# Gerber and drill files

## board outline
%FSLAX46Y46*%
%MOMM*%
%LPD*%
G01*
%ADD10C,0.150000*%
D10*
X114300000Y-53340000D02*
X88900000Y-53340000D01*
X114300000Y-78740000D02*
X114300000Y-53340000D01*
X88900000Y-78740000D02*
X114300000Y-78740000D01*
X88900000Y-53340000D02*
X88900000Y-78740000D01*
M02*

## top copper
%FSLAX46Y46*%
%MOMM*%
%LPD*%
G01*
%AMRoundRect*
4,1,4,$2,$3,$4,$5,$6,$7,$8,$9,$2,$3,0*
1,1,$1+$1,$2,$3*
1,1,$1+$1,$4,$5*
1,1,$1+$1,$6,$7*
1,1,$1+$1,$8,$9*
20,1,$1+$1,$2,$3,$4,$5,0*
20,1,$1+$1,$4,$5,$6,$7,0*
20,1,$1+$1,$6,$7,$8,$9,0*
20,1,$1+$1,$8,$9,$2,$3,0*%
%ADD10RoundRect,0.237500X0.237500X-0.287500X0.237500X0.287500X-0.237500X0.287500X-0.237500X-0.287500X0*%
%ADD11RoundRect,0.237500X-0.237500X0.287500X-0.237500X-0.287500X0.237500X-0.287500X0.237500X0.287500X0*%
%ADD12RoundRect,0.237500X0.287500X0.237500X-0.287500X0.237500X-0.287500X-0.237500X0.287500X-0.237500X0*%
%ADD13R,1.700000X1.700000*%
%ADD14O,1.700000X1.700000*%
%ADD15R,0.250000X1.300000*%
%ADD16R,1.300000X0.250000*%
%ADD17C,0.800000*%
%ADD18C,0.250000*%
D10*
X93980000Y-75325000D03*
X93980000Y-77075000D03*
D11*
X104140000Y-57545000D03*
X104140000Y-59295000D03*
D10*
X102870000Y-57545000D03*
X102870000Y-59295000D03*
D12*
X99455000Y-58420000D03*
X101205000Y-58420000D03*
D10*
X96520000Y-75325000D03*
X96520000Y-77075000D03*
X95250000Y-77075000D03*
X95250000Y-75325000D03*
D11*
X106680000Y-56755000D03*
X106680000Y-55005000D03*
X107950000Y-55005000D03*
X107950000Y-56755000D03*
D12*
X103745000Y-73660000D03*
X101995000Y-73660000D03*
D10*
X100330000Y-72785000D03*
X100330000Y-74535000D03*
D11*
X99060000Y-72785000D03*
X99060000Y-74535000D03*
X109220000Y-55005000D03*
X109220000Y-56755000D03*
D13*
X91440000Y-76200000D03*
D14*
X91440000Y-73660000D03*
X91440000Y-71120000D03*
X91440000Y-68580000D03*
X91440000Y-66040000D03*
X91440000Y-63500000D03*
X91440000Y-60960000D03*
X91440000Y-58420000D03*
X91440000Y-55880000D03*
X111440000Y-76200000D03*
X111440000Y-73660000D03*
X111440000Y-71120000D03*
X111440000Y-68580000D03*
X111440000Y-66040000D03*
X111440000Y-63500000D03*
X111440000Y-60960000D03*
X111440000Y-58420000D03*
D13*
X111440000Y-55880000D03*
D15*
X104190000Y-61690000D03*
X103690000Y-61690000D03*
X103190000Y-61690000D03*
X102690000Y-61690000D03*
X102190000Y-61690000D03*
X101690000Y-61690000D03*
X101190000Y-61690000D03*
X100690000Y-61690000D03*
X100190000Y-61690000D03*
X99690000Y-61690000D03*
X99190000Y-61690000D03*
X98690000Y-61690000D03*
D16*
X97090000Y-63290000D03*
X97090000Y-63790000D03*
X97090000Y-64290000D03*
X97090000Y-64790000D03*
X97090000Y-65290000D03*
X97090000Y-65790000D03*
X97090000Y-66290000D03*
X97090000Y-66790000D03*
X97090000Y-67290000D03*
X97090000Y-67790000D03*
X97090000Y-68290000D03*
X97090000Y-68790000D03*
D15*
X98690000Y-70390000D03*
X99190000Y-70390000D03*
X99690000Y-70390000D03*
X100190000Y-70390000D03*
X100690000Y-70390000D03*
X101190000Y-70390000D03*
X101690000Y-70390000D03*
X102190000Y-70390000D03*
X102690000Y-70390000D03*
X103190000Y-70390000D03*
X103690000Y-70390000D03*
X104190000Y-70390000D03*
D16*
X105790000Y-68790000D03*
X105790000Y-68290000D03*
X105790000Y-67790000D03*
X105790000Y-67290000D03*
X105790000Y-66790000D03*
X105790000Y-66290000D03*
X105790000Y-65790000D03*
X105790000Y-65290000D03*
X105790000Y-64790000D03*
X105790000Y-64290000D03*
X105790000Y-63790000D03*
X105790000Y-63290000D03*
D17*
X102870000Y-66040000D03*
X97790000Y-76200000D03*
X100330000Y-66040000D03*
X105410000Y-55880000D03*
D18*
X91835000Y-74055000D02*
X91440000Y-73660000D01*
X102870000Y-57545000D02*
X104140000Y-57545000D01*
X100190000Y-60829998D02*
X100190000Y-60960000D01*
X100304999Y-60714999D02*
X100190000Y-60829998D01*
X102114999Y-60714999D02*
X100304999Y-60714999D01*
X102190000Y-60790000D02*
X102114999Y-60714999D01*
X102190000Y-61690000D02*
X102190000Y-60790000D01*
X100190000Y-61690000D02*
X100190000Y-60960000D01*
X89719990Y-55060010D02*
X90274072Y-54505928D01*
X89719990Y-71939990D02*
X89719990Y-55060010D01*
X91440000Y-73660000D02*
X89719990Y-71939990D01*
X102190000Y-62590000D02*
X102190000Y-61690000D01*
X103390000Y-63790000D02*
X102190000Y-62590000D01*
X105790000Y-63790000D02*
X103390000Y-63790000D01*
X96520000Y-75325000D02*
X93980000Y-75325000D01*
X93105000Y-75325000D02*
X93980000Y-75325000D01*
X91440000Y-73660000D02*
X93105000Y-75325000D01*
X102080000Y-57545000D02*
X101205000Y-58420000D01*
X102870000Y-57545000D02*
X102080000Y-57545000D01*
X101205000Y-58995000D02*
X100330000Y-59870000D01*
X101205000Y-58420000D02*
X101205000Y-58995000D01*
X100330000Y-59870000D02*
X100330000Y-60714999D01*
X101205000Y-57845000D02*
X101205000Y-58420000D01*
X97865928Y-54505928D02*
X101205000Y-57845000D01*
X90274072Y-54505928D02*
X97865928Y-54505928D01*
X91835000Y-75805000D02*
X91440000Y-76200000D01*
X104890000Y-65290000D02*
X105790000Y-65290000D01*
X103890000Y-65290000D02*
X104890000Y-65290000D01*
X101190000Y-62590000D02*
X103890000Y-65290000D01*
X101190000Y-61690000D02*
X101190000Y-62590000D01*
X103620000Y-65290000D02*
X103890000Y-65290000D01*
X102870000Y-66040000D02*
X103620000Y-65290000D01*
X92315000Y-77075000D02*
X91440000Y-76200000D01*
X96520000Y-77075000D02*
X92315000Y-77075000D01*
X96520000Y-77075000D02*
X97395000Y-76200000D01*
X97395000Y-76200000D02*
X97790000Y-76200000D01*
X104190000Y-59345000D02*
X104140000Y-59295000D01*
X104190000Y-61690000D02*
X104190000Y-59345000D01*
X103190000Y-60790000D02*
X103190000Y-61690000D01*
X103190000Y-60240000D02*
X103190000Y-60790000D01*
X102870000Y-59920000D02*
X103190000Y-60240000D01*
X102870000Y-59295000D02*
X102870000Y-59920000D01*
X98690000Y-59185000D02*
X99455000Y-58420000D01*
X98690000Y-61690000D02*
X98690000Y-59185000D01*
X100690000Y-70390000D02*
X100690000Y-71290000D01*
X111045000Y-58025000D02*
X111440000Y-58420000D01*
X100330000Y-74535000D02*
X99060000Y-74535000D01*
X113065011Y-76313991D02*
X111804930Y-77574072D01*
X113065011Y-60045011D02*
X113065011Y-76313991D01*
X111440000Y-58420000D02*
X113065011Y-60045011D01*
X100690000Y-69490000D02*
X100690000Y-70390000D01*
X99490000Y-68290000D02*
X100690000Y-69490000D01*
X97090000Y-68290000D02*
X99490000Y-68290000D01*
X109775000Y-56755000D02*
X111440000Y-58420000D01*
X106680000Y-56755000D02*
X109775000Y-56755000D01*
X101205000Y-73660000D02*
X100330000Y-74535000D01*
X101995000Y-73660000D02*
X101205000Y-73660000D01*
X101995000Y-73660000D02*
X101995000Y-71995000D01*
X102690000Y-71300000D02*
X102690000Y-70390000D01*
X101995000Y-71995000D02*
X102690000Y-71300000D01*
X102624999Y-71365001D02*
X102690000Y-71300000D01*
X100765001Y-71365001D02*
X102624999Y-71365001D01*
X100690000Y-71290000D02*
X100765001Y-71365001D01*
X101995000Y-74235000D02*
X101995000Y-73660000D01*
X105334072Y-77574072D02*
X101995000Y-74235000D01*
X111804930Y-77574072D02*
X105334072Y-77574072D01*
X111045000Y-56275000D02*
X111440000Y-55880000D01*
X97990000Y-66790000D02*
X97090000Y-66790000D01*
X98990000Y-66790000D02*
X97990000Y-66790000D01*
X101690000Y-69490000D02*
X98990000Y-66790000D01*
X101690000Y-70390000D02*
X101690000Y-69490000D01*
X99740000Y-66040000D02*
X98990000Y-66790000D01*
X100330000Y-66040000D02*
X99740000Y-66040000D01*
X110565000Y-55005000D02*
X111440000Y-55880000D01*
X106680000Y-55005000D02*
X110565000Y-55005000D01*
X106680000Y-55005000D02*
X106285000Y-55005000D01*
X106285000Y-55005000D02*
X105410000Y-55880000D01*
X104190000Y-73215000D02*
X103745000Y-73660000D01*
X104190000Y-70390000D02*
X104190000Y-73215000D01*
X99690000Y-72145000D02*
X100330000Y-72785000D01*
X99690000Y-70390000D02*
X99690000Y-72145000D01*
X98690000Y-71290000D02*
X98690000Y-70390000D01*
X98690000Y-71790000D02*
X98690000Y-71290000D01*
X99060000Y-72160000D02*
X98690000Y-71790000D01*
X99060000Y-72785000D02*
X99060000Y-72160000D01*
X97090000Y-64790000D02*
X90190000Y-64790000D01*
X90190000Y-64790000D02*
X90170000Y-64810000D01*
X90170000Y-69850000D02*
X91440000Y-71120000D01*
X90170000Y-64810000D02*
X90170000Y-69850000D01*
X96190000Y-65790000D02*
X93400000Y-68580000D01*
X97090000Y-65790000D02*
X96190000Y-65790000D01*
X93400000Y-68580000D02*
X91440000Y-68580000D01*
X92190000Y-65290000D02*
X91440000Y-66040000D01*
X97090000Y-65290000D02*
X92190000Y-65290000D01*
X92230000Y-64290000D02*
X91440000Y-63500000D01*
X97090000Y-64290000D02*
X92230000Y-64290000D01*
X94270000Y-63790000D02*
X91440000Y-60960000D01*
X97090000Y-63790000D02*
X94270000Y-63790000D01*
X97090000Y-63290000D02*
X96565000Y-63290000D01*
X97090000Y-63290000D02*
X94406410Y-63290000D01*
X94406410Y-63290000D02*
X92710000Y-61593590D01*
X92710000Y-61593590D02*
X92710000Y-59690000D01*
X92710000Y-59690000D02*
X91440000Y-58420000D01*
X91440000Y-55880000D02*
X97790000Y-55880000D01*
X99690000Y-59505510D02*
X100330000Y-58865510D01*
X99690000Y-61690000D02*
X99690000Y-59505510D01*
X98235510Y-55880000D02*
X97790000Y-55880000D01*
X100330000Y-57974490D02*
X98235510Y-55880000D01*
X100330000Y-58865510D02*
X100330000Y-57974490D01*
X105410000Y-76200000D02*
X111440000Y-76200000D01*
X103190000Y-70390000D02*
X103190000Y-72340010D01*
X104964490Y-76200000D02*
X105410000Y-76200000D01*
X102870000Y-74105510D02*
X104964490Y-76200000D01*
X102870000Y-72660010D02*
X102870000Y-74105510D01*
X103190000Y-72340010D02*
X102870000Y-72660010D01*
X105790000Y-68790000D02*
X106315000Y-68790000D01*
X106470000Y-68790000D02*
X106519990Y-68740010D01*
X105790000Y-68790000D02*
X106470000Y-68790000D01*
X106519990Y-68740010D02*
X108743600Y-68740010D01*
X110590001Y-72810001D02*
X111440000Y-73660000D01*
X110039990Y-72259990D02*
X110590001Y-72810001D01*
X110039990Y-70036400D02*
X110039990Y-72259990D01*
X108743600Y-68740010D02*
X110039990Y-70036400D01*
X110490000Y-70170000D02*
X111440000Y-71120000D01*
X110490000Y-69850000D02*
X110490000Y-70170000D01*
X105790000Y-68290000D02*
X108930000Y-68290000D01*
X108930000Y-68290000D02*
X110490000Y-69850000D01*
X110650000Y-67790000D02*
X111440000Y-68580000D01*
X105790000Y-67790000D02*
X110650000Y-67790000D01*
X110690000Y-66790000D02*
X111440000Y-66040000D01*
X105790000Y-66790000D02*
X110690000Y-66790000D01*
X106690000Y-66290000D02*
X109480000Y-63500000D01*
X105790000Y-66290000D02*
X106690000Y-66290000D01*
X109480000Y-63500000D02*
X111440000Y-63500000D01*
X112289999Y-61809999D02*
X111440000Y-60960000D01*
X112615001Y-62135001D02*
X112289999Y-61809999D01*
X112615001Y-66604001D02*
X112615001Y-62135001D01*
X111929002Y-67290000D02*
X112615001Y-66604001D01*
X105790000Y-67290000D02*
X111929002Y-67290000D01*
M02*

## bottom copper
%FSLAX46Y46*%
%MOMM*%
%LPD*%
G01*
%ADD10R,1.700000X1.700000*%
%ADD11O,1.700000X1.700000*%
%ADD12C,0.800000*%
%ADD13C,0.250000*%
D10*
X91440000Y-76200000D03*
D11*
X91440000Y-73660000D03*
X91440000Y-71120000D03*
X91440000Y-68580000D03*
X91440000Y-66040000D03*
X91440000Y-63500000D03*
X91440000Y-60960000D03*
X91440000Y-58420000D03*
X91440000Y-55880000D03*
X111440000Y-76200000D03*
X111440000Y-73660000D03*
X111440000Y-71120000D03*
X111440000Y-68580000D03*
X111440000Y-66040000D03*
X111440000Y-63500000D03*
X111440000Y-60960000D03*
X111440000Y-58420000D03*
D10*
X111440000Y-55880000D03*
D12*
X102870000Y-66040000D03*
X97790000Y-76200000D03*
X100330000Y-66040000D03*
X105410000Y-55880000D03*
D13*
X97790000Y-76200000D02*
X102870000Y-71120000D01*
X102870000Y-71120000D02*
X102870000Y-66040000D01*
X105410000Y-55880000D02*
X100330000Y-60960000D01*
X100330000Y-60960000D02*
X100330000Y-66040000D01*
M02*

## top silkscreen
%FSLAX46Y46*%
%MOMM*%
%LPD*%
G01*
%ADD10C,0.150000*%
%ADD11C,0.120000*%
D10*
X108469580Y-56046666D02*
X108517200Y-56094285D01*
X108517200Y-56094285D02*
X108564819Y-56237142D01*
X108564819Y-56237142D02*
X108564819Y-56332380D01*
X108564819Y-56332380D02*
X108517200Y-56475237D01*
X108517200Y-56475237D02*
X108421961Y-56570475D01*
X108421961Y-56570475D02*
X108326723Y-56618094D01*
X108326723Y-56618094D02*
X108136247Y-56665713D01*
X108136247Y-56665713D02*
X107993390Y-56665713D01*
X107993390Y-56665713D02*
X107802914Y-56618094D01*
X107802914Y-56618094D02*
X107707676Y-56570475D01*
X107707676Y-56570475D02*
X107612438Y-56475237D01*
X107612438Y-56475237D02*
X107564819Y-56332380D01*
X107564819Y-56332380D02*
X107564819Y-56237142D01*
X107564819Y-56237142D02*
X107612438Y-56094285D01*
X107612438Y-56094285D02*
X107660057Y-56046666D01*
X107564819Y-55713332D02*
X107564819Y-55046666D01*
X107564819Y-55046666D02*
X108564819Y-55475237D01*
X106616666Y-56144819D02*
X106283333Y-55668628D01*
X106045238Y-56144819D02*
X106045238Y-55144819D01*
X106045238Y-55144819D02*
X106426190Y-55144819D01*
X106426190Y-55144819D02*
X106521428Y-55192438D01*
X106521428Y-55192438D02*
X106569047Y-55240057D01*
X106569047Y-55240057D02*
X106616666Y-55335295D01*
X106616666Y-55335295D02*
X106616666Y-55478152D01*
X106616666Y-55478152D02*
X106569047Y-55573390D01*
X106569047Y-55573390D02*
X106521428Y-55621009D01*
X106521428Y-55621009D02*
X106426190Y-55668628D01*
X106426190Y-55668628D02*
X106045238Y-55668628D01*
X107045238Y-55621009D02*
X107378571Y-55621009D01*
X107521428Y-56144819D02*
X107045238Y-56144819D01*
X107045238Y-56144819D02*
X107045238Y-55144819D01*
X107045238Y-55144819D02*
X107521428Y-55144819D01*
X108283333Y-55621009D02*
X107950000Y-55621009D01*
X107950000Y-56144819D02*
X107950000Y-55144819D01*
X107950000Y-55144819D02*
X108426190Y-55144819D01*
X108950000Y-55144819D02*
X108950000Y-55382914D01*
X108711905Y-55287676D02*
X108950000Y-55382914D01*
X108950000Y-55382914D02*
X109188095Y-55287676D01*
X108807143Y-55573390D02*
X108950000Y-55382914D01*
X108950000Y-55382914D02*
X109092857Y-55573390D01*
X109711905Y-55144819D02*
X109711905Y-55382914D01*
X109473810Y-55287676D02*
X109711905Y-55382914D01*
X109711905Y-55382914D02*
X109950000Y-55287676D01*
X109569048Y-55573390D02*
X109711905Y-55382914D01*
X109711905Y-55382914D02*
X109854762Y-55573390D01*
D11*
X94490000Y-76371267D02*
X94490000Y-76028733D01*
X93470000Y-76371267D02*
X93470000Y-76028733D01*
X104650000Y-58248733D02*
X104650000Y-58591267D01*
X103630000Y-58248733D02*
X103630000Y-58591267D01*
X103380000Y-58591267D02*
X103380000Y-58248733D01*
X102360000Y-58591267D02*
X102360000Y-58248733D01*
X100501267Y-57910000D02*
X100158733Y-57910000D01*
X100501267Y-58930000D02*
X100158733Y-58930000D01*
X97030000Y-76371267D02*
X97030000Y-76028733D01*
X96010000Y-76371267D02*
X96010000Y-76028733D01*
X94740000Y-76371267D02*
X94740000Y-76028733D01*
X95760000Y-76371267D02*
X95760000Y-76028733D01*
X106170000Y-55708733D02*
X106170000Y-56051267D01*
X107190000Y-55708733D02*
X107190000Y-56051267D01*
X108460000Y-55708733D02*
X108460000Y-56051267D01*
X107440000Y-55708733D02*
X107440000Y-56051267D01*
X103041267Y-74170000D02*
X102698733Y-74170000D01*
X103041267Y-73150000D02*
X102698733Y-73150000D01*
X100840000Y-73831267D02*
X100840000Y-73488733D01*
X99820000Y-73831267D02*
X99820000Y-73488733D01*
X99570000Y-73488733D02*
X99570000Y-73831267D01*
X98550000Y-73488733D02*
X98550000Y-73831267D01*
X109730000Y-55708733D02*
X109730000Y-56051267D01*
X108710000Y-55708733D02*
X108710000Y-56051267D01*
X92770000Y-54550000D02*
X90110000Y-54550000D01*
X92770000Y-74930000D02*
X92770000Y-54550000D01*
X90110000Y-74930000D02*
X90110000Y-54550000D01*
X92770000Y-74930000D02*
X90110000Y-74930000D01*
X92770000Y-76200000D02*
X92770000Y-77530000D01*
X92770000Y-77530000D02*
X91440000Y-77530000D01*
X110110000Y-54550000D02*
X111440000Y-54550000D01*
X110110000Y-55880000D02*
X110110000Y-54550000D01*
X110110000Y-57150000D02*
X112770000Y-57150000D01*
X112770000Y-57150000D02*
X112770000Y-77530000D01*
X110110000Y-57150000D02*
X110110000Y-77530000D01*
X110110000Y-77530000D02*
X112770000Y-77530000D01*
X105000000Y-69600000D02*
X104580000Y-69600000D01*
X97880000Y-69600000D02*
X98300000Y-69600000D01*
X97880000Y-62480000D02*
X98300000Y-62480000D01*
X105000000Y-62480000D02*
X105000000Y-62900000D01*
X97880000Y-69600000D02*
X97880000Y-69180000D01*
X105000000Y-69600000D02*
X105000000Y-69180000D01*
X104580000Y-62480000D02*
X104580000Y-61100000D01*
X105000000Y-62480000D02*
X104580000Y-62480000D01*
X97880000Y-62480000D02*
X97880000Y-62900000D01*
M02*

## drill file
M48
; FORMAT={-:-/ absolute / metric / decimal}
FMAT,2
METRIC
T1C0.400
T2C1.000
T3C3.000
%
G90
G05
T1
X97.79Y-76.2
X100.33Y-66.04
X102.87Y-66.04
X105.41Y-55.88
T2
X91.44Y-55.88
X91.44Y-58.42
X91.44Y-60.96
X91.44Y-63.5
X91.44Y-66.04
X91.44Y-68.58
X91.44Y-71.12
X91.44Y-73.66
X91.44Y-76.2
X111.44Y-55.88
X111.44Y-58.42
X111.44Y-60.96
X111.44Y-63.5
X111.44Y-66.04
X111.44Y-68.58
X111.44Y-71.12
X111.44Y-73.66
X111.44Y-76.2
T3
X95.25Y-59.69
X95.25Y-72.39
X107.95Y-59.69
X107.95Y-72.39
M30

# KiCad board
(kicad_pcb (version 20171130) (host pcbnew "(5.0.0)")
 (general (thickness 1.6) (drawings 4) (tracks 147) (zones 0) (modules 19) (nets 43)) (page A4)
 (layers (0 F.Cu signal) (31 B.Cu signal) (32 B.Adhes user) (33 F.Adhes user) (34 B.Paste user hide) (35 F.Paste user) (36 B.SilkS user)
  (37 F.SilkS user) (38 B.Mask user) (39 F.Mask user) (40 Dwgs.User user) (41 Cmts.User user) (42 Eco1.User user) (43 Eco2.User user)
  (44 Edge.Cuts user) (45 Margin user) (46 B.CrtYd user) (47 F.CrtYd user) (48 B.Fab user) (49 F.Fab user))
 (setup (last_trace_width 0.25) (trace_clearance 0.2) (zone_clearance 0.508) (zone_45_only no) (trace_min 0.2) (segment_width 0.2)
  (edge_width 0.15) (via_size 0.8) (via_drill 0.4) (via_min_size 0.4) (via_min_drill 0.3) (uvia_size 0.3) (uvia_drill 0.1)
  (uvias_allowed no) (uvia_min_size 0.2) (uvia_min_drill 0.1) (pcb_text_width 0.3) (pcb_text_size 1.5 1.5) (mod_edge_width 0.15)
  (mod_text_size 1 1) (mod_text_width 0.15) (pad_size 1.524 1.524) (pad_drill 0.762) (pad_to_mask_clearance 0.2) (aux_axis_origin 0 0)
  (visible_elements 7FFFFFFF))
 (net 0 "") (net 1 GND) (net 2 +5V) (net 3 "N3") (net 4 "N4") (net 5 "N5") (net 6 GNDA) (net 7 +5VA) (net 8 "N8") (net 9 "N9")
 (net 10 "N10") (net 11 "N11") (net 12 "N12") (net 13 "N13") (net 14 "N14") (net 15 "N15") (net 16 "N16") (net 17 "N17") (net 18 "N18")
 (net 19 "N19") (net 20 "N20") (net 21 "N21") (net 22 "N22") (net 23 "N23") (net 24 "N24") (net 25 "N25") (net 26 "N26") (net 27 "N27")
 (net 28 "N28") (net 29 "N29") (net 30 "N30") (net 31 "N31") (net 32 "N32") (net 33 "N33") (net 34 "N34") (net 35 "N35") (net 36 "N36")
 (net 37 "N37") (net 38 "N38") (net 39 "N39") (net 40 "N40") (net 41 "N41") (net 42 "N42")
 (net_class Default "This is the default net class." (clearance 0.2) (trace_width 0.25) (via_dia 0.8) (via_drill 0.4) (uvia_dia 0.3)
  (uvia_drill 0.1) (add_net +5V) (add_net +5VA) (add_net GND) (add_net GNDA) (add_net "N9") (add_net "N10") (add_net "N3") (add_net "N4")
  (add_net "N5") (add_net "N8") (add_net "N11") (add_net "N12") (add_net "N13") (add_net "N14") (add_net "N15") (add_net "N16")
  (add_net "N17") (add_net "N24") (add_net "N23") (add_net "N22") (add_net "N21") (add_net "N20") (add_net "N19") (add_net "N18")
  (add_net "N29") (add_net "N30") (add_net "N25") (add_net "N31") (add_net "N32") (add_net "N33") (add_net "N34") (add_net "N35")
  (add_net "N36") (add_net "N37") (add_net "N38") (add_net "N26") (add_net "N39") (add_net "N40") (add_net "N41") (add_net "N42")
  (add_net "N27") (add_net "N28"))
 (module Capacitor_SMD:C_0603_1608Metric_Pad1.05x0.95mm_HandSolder (layer F.Cu) (at 93.98 76.2 90)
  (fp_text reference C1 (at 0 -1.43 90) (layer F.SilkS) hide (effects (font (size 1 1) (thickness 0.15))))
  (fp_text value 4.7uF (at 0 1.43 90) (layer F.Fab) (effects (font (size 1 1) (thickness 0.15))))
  (fp_line (start -0.171267 0.51) (end 0.171267 0.51) (layer F.SilkS) (width 0.12))
  (fp_line (start -0.171267 -0.51) (end 0.171267 -0.51) (layer F.SilkS) (width 0.12))
  (pad 2 smd roundrect (at 0.875 0 90) (size 1.05 0.95) (layers F.Cu F.Paste F.Mask) (roundrect_rratio 0.25) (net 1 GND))
  (pad 1 smd roundrect (at -0.875 0 90) (size 1.05 0.95) (layers F.Cu F.Paste F.Mask) (roundrect_rratio 0.25) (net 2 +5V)))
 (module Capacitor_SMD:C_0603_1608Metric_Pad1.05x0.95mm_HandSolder (layer F.Cu) (at 104.14 58.42 270)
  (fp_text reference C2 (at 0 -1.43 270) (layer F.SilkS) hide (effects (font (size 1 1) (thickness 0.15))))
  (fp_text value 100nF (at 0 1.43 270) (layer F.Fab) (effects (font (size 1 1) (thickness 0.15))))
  (fp_line (start -0.171267 -0.51) (end 0.171267 -0.51) (layer F.SilkS) (width 0.12))
  (fp_line (start -0.171267 0.51) (end 0.171267 0.51) (layer F.SilkS) (width 0.12))
  (pad 1 smd roundrect (at -0.875 0 270) (size 1.05 0.95) (layers F.Cu F.Paste F.Mask) (roundrect_rratio 0.25) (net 1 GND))
  (pad 2 smd roundrect (at 0.875 0 270) (size 1.05 0.95) (layers F.Cu F.Paste F.Mask) (roundrect_rratio 0.25) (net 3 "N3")))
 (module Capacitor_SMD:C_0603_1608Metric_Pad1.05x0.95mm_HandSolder (layer F.Cu) (at 102.87 58.42 90)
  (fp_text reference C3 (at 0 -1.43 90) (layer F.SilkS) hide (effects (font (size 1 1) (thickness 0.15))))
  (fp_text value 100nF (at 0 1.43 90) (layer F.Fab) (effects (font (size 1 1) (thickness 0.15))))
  (fp_line (start -0.171267 0.51) (end 0.171267 0.51) (layer F.SilkS) (width 0.12))
  (fp_line (start -0.171267 -0.51) (end 0.171267 -0.51) (layer F.SilkS) (width 0.12))
  (pad 2 smd roundrect (at 0.875 0 90) (size 1.05 0.95) (layers F.Cu F.Paste F.Mask) (roundrect_rratio 0.25) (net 1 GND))
  (pad 1 smd roundrect (at -0.875 0 90) (size 1.05 0.95) (layers F.Cu F.Paste F.Mask) (roundrect_rratio 0.25) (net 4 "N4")))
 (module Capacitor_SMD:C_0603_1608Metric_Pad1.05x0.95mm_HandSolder (layer F.Cu) (at 100.33 58.42 180)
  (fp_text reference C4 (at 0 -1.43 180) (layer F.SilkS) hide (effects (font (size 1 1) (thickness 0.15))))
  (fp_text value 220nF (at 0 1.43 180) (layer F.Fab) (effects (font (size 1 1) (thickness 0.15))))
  (fp_line (start -0.171267 0.51) (end 0.171267 0.51) (layer F.SilkS) (width 0.12))
  (fp_line (start -0.171267 -0.51) (end 0.171267 -0.51) (layer F.SilkS) (width 0.12))
  (pad 2 smd roundrect (at 0.875 0 180) (size 1.05 0.95) (layers F.Cu F.Paste F.Mask) (roundrect_rratio 0.25) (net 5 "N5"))
  (pad 1 smd roundrect (at -0.875 0 180) (size 1.05 0.95) (layers F.Cu F.Paste F.Mask) (roundrect_rratio 0.25) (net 1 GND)))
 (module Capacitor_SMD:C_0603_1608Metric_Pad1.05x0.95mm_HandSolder (layer F.Cu) (at 96.52 76.2 90)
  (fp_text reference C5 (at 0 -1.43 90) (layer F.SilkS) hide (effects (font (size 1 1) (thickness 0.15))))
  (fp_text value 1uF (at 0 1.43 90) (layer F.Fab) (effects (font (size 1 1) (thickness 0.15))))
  (fp_line (start -0.171267 0.51) (end 0.171267 0.51) (layer F.SilkS) (width 0.12))
  (fp_line (start -0.171267 -0.51) (end 0.171267 -0.51) (layer F.SilkS) (width 0.12))
  (pad 2 smd roundrect (at 0.875 0 90) (size 1.05 0.95) (layers F.Cu F.Paste F.Mask) (roundrect_rratio 0.25) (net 1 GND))
  (pad 1 smd roundrect (at -0.875 0 90) (size 1.05 0.95) (layers F.Cu F.Paste F.Mask) (roundrect_rratio 0.25) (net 2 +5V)))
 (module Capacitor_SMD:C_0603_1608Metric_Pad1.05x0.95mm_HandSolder (layer F.Cu) (at 95.25 76.2 90)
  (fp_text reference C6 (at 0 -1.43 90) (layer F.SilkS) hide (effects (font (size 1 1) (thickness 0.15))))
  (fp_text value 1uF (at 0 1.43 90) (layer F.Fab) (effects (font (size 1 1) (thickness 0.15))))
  (fp_line (start -0.171267 -0.51) (end 0.171267 -0.51) (layer F.SilkS) (width 0.12))
  (fp_line (start -0.171267 0.51) (end 0.171267 0.51) (layer F.SilkS) (width 0.12))
  (pad 1 smd roundrect (at -0.875 0 90) (size 1.05 0.95) (layers F.Cu F.Paste F.Mask) (roundrect_rratio 0.25) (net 2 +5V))
  (pad 2 smd roundrect (at 0.875 0 90) (size 1.05 0.95) (layers F.Cu F.Paste F.Mask) (roundrect_rratio 0.25) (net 1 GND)))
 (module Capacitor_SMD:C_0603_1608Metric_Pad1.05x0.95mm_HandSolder (layer F.Cu) (at 106.68 55.88 270)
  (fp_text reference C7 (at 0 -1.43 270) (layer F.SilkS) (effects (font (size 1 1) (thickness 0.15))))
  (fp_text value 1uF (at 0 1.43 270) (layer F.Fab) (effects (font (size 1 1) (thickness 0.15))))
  (fp_line (start -0.171267 0.51) (end 0.171267 0.51) (layer F.SilkS) (width 0.12))
  (fp_line (start -0.171267 -0.51) (end 0.171267 -0.51) (layer F.SilkS) (width 0.12))
  (pad 2 smd roundrect (at 0.875 0 270) (size 1.05 0.95) (layers F.Cu F.Paste F.Mask) (roundrect_rratio 0.25) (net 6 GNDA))
  (pad 1 smd roundrect (at -0.875 0 270) (size 1.05 0.95) (layers F.Cu F.Paste F.Mask) (roundrect_rratio 0.25) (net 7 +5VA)))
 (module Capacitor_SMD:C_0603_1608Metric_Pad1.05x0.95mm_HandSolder (layer F.Cu) (at 107.95 55.88 270)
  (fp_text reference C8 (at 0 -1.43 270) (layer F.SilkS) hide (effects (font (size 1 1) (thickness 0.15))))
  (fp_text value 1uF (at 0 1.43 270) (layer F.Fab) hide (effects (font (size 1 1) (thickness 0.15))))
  (fp_line (start -0.171267 -0.51) (end 0.171267 -0.51) (layer F.SilkS) (width 0.12))
  (fp_line (start -0.171267 0.51) (end 0.171267 0.51) (layer F.SilkS) (width 0.12))
  (pad 1 smd roundrect (at -0.875 0 270) (size 1.05 0.95) (layers F.Cu F.Paste F.Mask) (roundrect_rratio 0.25) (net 7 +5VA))
  (pad 2 smd roundrect (at 0.875 0 270) (size 1.05 0.95) (layers F.Cu F.Paste F.Mask) (roundrect_rratio 0.25) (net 6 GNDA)))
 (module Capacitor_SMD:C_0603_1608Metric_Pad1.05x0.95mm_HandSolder (layer F.Cu) (at 102.87 73.66 180)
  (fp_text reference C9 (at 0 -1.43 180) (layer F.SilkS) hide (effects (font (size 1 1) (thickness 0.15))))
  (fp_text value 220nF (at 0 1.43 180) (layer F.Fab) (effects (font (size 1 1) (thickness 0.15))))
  (fp_line (start -0.171267 -0.51) (end 0.171267 -0.51) (layer F.SilkS) (width 0.12))
  (fp_line (start -0.171267 0.51) (end 0.171267 0.51) (layer F.SilkS) (width 0.12))
  (pad 1 smd roundrect (at -0.875 0 180) (size 1.05 0.95) (layers F.Cu F.Paste F.Mask) (roundrect_rratio 0.25) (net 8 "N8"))
  (pad 2 smd roundrect (at 0.875 0 180) (size 1.05 0.95) (layers F.Cu F.Paste F.Mask) (roundrect_rratio 0.25) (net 6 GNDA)))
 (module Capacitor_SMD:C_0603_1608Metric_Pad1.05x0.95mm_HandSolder (layer F.Cu) (at 100.33 73.66 90)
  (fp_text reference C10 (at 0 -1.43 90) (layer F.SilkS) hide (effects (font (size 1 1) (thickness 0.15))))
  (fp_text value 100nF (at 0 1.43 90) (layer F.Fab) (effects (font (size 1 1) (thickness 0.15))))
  (fp_line (start -0.171267 0.51) (end 0.171267 0.51) (layer F.SilkS) (width 0.12))
  (fp_line (start -0.171267 -0.51) (end 0.171267 -0.51) (layer F.SilkS) (width 0.12))
  (pad 2 smd roundrect (at 0.875 0 90) (size 1.05 0.95) (layers F.Cu F.Paste F.Mask) (roundrect_rratio 0.25) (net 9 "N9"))
  (pad 1 smd roundrect (at -0.875 0 90) (size 1.05 0.95) (layers F.Cu F.Paste F.Mask) (roundrect_rratio 0.25) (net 6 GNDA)))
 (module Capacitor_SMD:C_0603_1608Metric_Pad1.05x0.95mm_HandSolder (layer F.Cu) (at 99.06 73.66 270)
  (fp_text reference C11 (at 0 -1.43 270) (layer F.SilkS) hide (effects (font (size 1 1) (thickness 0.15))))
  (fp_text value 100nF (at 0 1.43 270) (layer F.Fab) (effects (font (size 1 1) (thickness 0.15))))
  (fp_line (start -0.171267 -0.51) (end 0.171267 -0.51) (layer F.SilkS) (width 0.12))
  (fp_line (start -0.171267 0.51) (end 0.171267 0.51) (layer F.SilkS) (width 0.12))
  (pad 1 smd roundrect (at -0.875 0 270) (size 1.05 0.95) (layers F.Cu F.Paste F.Mask) (roundrect_rratio 0.25) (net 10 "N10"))
  (pad 2 smd roundrect (at 0.875 0 270) (size 1.05 0.95) (layers F.Cu F.Paste F.Mask) (roundrect_rratio 0.25) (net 6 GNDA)))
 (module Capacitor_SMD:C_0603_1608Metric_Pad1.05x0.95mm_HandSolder (layer F.Cu) (at 109.22 55.88 270)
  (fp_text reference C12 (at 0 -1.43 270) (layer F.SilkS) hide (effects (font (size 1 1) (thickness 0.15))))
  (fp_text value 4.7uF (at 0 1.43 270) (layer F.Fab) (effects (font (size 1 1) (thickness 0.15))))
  (fp_line (start -0.171267 -0.51) (end 0.171267 -0.51) (layer F.SilkS) (width 0.12))
  (fp_line (start -0.171267 0.51) (end 0.171267 0.51) (layer F.SilkS) (width 0.12))
  (pad 1 smd roundrect (at -0.875 0 270) (size 1.05 0.95) (layers F.Cu F.Paste F.Mask) (roundrect_rratio 0.25) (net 7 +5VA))
  (pad 2 smd roundrect (at 0.875 0 270) (size 1.05 0.95) (layers F.Cu F.Paste F.Mask) (roundrect_rratio 0.25) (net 6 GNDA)))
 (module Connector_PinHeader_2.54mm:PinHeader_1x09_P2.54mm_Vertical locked (layer F.Cu) (at 91.44 76.2 180)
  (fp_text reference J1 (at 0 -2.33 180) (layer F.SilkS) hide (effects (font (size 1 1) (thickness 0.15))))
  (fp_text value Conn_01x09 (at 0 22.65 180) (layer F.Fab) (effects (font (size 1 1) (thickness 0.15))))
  (fp_line (start -1.33 21.65) (end 1.33 21.65) (layer F.SilkS) (width 0.12))
  (fp_line (start -1.33 1.27) (end -1.33 21.65) (layer F.SilkS) (width 0.12))
  (fp_line (start 1.33 1.27) (end 1.33 21.65) (layer F.SilkS) (width 0.12))
  (fp_line (start -1.33 1.27) (end 1.33 1.27) (layer F.SilkS) (width 0.12))
  (fp_line (start -1.33 0) (end -1.33 -1.33) (layer F.SilkS) (width 0.12))
  (fp_line (start -1.33 -1.33) (end 0 -1.33) (layer F.SilkS) (width 0.12))
  (pad 1 thru_hole rect (at 0 0 180) (size 1.7 1.7) (drill 1) (layers *.Cu *.Mask) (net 2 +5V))
  (pad 2 thru_hole oval (at 0 2.54 180) (size 1.7 1.7) (drill 1) (layers *.Cu *.Mask) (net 1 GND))
  (pad 3 thru_hole oval (at 0 5.08 180) (size 1.7 1.7) (drill 1) (layers *.Cu *.Mask) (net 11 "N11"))
  (pad 4 thru_hole oval (at 0 7.62 180) (size 1.7 1.7) (drill 1) (layers *.Cu *.Mask) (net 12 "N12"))
  (pad 5 thru_hole oval (at 0 10.16 180) (size 1.7 1.7) (drill 1) (layers *.Cu *.Mask) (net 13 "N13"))
  (pad 6 thru_hole oval (at 0 12.7 180) (size 1.7 1.7) (drill 1) (layers *.Cu *.Mask) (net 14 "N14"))
  (pad 7 thru_hole oval (at 0 15.24 180) (size 1.7 1.7) (drill 1) (layers *.Cu *.Mask) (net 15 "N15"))
  (pad 8 thru_hole oval (at 0 17.78 180) (size 1.7 1.7) (drill 1) (layers *.Cu *.Mask) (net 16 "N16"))
  (pad 9 thru_hole oval (at 0 20.32 180) (size 1.7 1.7) (drill 1) (layers *.Cu *.Mask) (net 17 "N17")))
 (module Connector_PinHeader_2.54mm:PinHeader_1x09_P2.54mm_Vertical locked (layer F.Cu) (at 111.44 55.88)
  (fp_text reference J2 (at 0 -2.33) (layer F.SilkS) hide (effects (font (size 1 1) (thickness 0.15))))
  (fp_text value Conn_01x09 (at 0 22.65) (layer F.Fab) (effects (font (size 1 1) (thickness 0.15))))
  (fp_line (start -1.33 -1.33) (end 0 -1.33) (layer F.SilkS) (width 0.12))
  (fp_line (start -1.33 0) (end -1.33 -1.33) (layer F.SilkS) (width 0.12))
  (fp_line (start -1.33 1.27) (end 1.33 1.27) (layer F.SilkS) (width 0.12))
  (fp_line (start 1.33 1.27) (end 1.33 21.65) (layer F.SilkS) (width 0.12))
  (fp_line (start -1.33 1.27) (end -1.33 21.65) (layer F.SilkS) (width 0.12))
  (fp_line (start -1.33 21.65) (end 1.33 21.65) (layer F.SilkS) (width 0.12))
  (pad 9 thru_hole oval (at 0 20.32) (size 1.7 1.7) (drill 1) (layers *.Cu *.Mask) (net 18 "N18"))
  (pad 8 thru_hole oval (at 0 17.78) (size 1.7 1.7) (drill 1) (layers *.Cu *.Mask) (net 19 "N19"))
  (pad 7 thru_hole oval (at 0 15.24) (size 1.7 1.7) (drill 1) (layers *.Cu *.Mask) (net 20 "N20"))
  (pad 6 thru_hole oval (at 0 12.7) (size 1.7 1.7) (drill 1) (layers *.Cu *.Mask) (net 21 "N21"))
  (pad 5 thru_hole oval (at 0 10.16) (size 1.7 1.7) (drill 1) (layers *.Cu *.Mask) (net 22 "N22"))
  (pad 4 thru_hole oval (at 0 7.62) (size 1.7 1.7) (drill 1) (layers *.Cu *.Mask) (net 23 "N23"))
  (pad 3 thru_hole oval (at 0 5.08) (size 1.7 1.7) (drill 1) (layers *.Cu *.Mask) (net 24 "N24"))
  (pad 2 thru_hole oval (at 0 2.54) (size 1.7 1.7) (drill 1) (layers *.Cu *.Mask) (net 6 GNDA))
  (pad 1 thru_hole rect (at 0 0) (size 1.7 1.7) (drill 1) (layers *.Cu *.Mask) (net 7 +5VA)))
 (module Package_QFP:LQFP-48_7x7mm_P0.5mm (layer F.Cu) (at 101.44 66.04 270)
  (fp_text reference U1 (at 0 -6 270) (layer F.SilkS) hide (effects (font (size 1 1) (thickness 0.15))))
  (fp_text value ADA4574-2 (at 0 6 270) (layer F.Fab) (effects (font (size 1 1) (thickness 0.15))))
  (fp_line (start 3.56 -3.56) (end 3.56 -3.14) (layer F.SilkS) (width 0.12))
  (fp_line (start 3.56 3.56) (end 3.56 3.14) (layer F.SilkS) (width 0.12))
  (fp_line (start -3.56 3.56) (end -3.56 3.14) (layer F.SilkS) (width 0.12))
  (fp_line (start -3.56 -3.56) (end -3.14 -3.56) (layer F.SilkS) (width 0.12))
  (fp_line (start 3.56 3.56) (end 3.14 3.56) (layer F.SilkS) (width 0.12))
  (fp_line (start 3.56 -3.56) (end 3.14 -3.56) (layer F.SilkS) (width 0.12))
  (fp_line (start -3.56 -3.14) (end -4.94 -3.14) (layer F.SilkS) (width 0.12))
  (fp_line (start -3.56 -3.56) (end -3.56 -3.14) (layer F.SilkS) (width 0.12))
  (fp_line (start -3.56 3.56) (end -3.14 3.56) (layer F.SilkS) (width 0.12))
  (pad 1 smd rect (at -4.35 -2.75 270) (size 1.3 0.25) (layers F.Cu F.Paste F.Mask) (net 3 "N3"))
  (pad 2 smd rect (at -4.35 -2.25 270) (size 1.3 0.25) (layers F.Cu F.Paste F.Mask) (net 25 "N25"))
  (pad 3 smd rect (at -4.35 -1.75 270) (size 1.3 0.25) (layers F.Cu F.Paste F.Mask) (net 4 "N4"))
  (pad 4 smd rect (at -4.35 -1.25 270) (size 1.3 0.25) (layers F.Cu F.Paste F.Mask) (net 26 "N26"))
  (pad 5 smd rect (at -4.35 -0.75 270) (size 1.3 0.25) (layers F.Cu F.Paste F.Mask) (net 1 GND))
  (pad 6 smd rect (at -4.35 -0.25 270) (size 1.3 0.25) (layers F.Cu F.Paste F.Mask) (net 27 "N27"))
  (pad 7 smd rect (at -4.35 0.25 270) (size 1.3 0.25) (layers F.Cu F.Paste F.Mask) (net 2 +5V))
  (pad 8 smd rect (at -4.35 0.75 270) (size 1.3 0.25) (layers F.Cu F.Paste F.Mask) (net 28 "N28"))
  (pad 9 smd rect (at -4.35 1.25 270) (size 1.3 0.25) (layers F.Cu F.Paste F.Mask) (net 1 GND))
  (pad 10 smd rect (at -4.35 1.75 270) (size 1.3 0.25) (layers F.Cu F.Paste F.Mask) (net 17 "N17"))
  (pad 11 smd rect (at -4.35 2.25 270) (size 1.3 0.25) (layers F.Cu F.Paste F.Mask) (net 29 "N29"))
  (pad 12 smd rect (at -4.35 2.75 270) (size 1.3 0.25) (layers F.Cu F.Paste F.Mask) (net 5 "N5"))
  (pad 13 smd rect (at -2.75 4.35) (size 1.3 0.25) (layers F.Cu F.Paste F.Mask) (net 16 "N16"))
  (pad 14 smd rect (at -2.25 4.35) (size 1.3 0.25) (layers F.Cu F.Paste F.Mask) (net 15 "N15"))
  (pad 15 smd rect (at -1.75 4.35) (size 1.3 0.25) (layers F.Cu F.Paste F.Mask) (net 14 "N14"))
  (pad 16 smd rect (at -1.25 4.35) (size 1.3 0.25) (layers F.Cu F.Paste F.Mask) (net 11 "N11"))
  (pad 17 smd rect (at -0.75 4.35) (size 1.3 0.25) (layers F.Cu F.Paste F.Mask) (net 13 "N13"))
  (pad 18 smd rect (at -0.25 4.35) (size 1.3 0.25) (layers F.Cu F.Paste F.Mask) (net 12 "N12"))
  (pad 19 smd rect (at 0.25 4.35) (size 1.3 0.25) (layers F.Cu F.Paste F.Mask) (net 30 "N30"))
  (pad 20 smd rect (at 0.75 4.35) (size 1.3 0.25) (layers F.Cu F.Paste F.Mask) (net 7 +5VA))
  (pad 21 smd rect (at 1.25 4.35) (size 1.3 0.25) (layers F.Cu F.Paste F.Mask) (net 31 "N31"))
  (pad 22 smd rect (at 1.75 4.35) (size 1.3 0.25) (layers F.Cu F.Paste F.Mask) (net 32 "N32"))
  (pad 23 smd rect (at 2.25 4.35) (size 1.3 0.25) (layers F.Cu F.Paste F.Mask) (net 6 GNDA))
  (pad 24 smd rect (at 2.75 4.35) (size 1.3 0.25) (layers F.Cu F.Paste F.Mask) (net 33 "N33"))
  (pad 25 smd rect (at 4.35 2.75 270) (size 1.3 0.25) (layers F.Cu F.Paste F.Mask) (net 10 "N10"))
  (pad 26 smd rect (at 4.35 2.25 270) (size 1.3 0.25) (layers F.Cu F.Paste F.Mask) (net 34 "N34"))
  (pad 27 smd rect (at 4.35 1.75 270) (size 1.3 0.25) (layers F.Cu F.Paste F.Mask) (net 9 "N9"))
  (pad 28 smd rect (at 4.35 1.25 270) (size 1.3 0.25) (layers F.Cu F.Paste F.Mask) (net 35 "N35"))
  (pad 29 smd rect (at 4.35 0.75 270) (size 1.3 0.25) (layers F.Cu F.Paste F.Mask) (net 6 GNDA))
  (pad 30 smd rect (at 4.35 0.25 270) (size 1.3 0.25) (layers F.Cu F.Paste F.Mask) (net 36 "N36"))
  (pad 31 smd rect (at 4.35 -0.25 270) (size 1.3 0.25) (layers F.Cu F.Paste F.Mask) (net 7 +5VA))
  (pad 32 smd rect (at 4.35 -0.75 270) (size 1.3 0.25) (layers F.Cu F.Paste F.Mask) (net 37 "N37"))
  (pad 33 smd rect (at 4.35 -1.25 270) (size 1.3 0.25) (layers F.Cu F.Paste F.Mask) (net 6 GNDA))
  (pad 34 smd rect (at 4.35 -1.75 270) (size 1.3 0.25) (layers F.Cu F.Paste F.Mask) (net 18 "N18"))
  (pad 35 smd rect (at 4.35 -2.25 270) (size 1.3 0.25) (layers F.Cu F.Paste F.Mask) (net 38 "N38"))
  (pad 36 smd rect (at 4.35 -2.75 270) (size 1.3 0.25) (layers F.Cu F.Paste F.Mask) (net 8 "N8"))
  (pad 37 smd rect (at 2.75 -4.35) (size 1.3 0.25) (layers F.Cu F.Paste F.Mask) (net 19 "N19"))
  (pad 38 smd rect (at 2.25 -4.35) (size 1.3 0.25) (layers F.Cu F.Paste F.Mask) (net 20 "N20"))
  (pad 39 smd rect (at 1.75 -4.35) (size 1.3 0.25) (layers F.Cu F.Paste F.Mask) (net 21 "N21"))
  (pad 40 smd rect (at 1.25 -4.35) (size 1.3 0.25) (layers F.Cu F.Paste F.Mask) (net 24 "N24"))
  (pad 41 smd rect (at 0.75 -4.35) (size 1.3 0.25) (layers F.Cu F.Paste F.Mask) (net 22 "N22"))
  (pad 42 smd rect (at 0.25 -4.35) (size 1.3 0.25) (layers F.Cu F.Paste F.Mask) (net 23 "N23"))
  (pad 43 smd rect (at -0.25 -4.35) (size 1.3 0.25) (layers F.Cu F.Paste F.Mask) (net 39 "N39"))
  (pad 44 smd rect (at -0.75 -4.35) (size 1.3 0.25) (layers F.Cu F.Paste F.Mask) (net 2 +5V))
  (pad 45 smd rect (at -1.25 -4.35) (size 1.3 0.25) (layers F.Cu F.Paste F.Mask) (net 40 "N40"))
  (pad 46 smd rect (at -1.75 -4.35) (size 1.3 0.25) (layers F.Cu F.Paste F.Mask) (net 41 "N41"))
  (pad 47 smd rect (at -2.25 -4.35) (size 1.3 0.25) (layers F.Cu F.Paste F.Mask) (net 1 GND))
  (pad 48 smd rect (at -2.75 -4.35) (size 1.3 0.25) (layers F.Cu F.Paste F.Mask) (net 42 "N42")))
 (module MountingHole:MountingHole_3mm (layer F.Cu) (at 107.95 59.69)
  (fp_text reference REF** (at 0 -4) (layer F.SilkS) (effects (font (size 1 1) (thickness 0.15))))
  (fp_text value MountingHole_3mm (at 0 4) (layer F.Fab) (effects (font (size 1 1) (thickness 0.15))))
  (pad 1 np_thru_hole circle (at 0 0) (size 3 3) (drill 3) (layers *.Cu *.Mask)))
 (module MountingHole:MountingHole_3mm (layer F.Cu) (at 95.25 72.39)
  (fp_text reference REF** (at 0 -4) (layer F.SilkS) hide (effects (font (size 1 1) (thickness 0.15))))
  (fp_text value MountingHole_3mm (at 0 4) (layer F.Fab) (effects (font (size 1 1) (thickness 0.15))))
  (pad 1 np_thru_hole circle (at 0 0) (size 3 3) (drill 3) (layers *.Cu *.Mask)))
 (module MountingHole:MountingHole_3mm (layer F.Cu) (at 107.95 72.39)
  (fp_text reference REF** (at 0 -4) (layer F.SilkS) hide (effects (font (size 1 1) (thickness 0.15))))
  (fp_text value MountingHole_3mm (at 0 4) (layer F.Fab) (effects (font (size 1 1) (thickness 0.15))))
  (pad 1 np_thru_hole circle (at 0 0) (size 3 3) (drill 3) (layers *.Cu *.Mask)))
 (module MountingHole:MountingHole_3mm (layer F.Cu) (at 95.25 59.69)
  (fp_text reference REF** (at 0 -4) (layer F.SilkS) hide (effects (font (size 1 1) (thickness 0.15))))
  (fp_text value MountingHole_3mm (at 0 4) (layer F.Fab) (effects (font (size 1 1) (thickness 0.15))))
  (pad 1 np_thru_hole circle (at 0 0) (size 3 3) (drill 3) (layers *.Cu *.Mask)))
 (gr_line (start 114.3 53.34) (end 88.9 53.34) (layer Edge.Cuts) (width 0.15))
 (gr_line (start 114.3 78.74) (end 114.3 53.34) (layer Edge.Cuts) (width 0.15))
 (gr_line (start 88.9 78.74) (end 114.3 78.74) (layer Edge.Cuts) (width 0.15))
 (gr_line (start 88.9 53.34) (end 88.9 78.74) (layer Edge.Cuts) (width 0.15))
 (segment (start 91.835 74.055) (end 91.44 73.66) (width 0.25) (layer F.Cu) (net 1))
 (segment (start 102.87 57.545) (end 104.14 57.545) (width 0.25) (layer F.Cu) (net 1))
 (segment (start 100.19 60.829998) (end 100.19 60.96) (width 0.25) (layer F.Cu) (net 1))
 (segment (start 100.304999 60.714999) (end 100.19 60.829998) (width 0.25) (layer F.Cu) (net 1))
 (segment (start 102.114999 60.714999) (end 100.304999 60.714999) (width 0.25) (layer F.Cu) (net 1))
 (segment (start 102.19 60.79) (end 102.114999 60.714999) (width 0.25) (layer F.Cu) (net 1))
 (segment (start 102.19 61.69) (end 102.19 60.79) (width 0.25) (layer F.Cu) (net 1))
 (segment (start 100.19 61.69) (end 100.19 60.96) (width 0.25) (layer F.Cu) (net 1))
 (segment (start 89.71999 55.06001) (end 90.274072 54.505928) (width 0.25) (layer F.Cu) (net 1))
 (segment (start 89.71999 71.93999) (end 89.71999 55.06001) (width 0.25) (layer F.Cu) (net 1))
 (segment (start 91.44 73.66) (end 89.71999 71.93999) (width 0.25) (layer F.Cu) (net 1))
 (segment (start 102.19 62.59) (end 102.19 61.69) (width 0.25) (layer F.Cu) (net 1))
 (segment (start 103.39 63.79) (end 102.19 62.59) (width 0.25) (layer F.Cu) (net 1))
 (segment (start 105.79 63.79) (end 103.39 63.79) (width 0.25) (layer F.Cu) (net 1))
 (segment (start 96.52 75.325) (end 93.98 75.325) (width 0.25) (layer F.Cu) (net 1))
 (segment (start 93.105 75.325) (end 93.98 75.325) (width 0.25) (layer F.Cu) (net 1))
 (segment (start 91.44 73.66) (end 93.105 75.325) (width 0.25) (layer F.Cu) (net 1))
 (segment (start 102.08 57.545) (end 101.205 58.42) (width 0.25) (layer F.Cu) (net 1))
 (segment (start 102.87 57.545) (end 102.08 57.545) (width 0.25) (layer F.Cu) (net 1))
 (segment (start 101.205 58.995) (end 100.33 59.87) (width 0.25) (layer F.Cu) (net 1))
 (segment (start 101.205 58.42) (end 101.205 58.995) (width 0.25) (layer F.Cu) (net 1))
 (segment (start 100.33 59.87) (end 100.33 60.714999) (width 0.25) (layer F.Cu) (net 1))
 (segment (start 101.205 57.845) (end 101.205 58.42) (width 0.25) (layer F.Cu) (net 1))
 (segment (start 97.865928 54.505928) (end 101.205 57.845) (width 0.25) (layer F.Cu) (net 1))
 (segment (start 90.274072 54.505928) (end 97.865928 54.505928) (width 0.25) (layer F.Cu) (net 1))
 (segment (start 91.835 75.805) (end 91.44 76.2) (width 0.25) (layer F.Cu) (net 2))
 (segment (start 104.89 65.29) (end 105.79 65.29) (width 0.25) (layer F.Cu) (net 2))
 (segment (start 103.89 65.29) (end 104.89 65.29) (width 0.25) (layer F.Cu) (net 2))
 (segment (start 101.19 62.59) (end 103.89 65.29) (width 0.25) (layer F.Cu) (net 2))
 (segment (start 101.19 61.69) (end 101.19 62.59) (width 0.25) (layer F.Cu) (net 2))
 (segment (start 97.79 76.2) (end 102.87 71.12) (width 0.25) (layer B.Cu) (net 2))
 (via (at 102.87 66.04) (size 0.8) (drill 0.4) (layers F.Cu B.Cu) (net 2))
 (segment (start 102.87 71.12) (end 102.87 66.04) (width 0.25) (layer B.Cu) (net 2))
 (segment (start 103.62 65.29) (end 103.89 65.29) (width 0.25) (layer F.Cu) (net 2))
 (segment (start 102.87 66.04) (end 103.62 65.29) (width 0.25) (layer F.Cu) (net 2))
 (segment (start 92.315 77.075) (end 91.44 76.2) (width 0.25) (layer F.Cu) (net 2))
 (segment (start 96.52 77.075) (end 92.315 77.075) (width 0.25) (layer F.Cu) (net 2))
 (segment (start 96.52 77.075) (end 97.395 76.2) (width 0.25) (layer F.Cu) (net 2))
 (via (at 97.79 76.2) (size 0.8) (drill 0.4) (layers F.Cu B.Cu) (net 2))
 (segment (start 97.395 76.2) (end 97.79 76.2) (width 0.25) (layer F.Cu) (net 2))
 (segment (start 104.19 59.345) (end 104.14 59.295) (width 0.25) (layer F.Cu) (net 3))
 (segment (start 104.19 61.69) (end 104.19 59.345) (width 0.25) (layer F.Cu) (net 3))
 (segment (start 103.19 60.79) (end 103.19 61.69) (width 0.25) (layer F.Cu) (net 4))
 (segment (start 103.19 60.24) (end 103.19 60.79) (width 0.25) (layer F.Cu) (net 4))
 (segment (start 102.87 59.92) (end 103.19 60.24) (width 0.25) (layer F.Cu) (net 4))
 (segment (start 102.87 59.295) (end 102.87 59.92) (width 0.25) (layer F.Cu) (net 4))
 (segment (start 98.69 59.185) (end 99.455 58.42) (width 0.25) (layer F.Cu) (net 5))
 (segment (start 98.69 61.69) (end 98.69 59.185) (width 0.25) (layer F.Cu) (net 5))
 (segment (start 100.69 70.39) (end 100.69 71.29) (width 0.25) (layer F.Cu) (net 6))
 (segment (start 111.045 58.025) (end 111.44 58.42) (width 0.25) (layer F.Cu) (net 6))
 (segment (start 100.33 74.535) (end 99.06 74.535) (width 0.25) (layer F.Cu) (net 6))
 (segment (start 113.065011 76.313991) (end 111.80493 77.574072) (width 0.25) (layer F.Cu) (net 6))
 (segment (start 113.065011 60.045011) (end 113.065011 76.313991) (width 0.25) (layer F.Cu) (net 6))
 (segment (start 111.44 58.42) (end 113.065011 60.045011) (width 0.25) (layer F.Cu) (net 6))
 (segment (start 100.69 69.49) (end 100.69 70.39) (width 0.25) (layer F.Cu) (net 6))
 (segment (start 99.49 68.29) (end 100.69 69.49) (width 0.25) (layer F.Cu) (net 6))
 (segment (start 97.09 68.29) (end 99.49 68.29) (width 0.25) (layer F.Cu) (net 6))
 (segment (start 109.775 56.755) (end 111.44 58.42) (width 0.25) (layer F.Cu) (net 6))
 (segment (start 106.68 56.755) (end 109.775 56.755) (width 0.25) (layer F.Cu) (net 6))
 (segment (start 101.205 73.66) (end 100.33 74.535) (width 0.25) (layer F.Cu) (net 6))
 (segment (start 101.995 73.66) (end 101.205 73.66) (width 0.25) (layer F.Cu) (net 6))
 (segment (start 101.995 73.66) (end 101.995 71.995) (width 0.25) (layer F.Cu) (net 6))
 (segment (start 102.69 71.3) (end 102.69 70.39) (width 0.25) (layer F.Cu) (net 6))
 (segment (start 101.995 71.995) (end 102.69 71.3) (width 0.25) (layer F.Cu) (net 6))
 (segment (start 102.624999 71.365001) (end 102.69 71.3) (width 0.25) (layer F.Cu) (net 6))
 (segment (start 100.765001 71.365001) (end 102.624999 71.365001) (width 0.25) (layer F.Cu) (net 6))
 (segment (start 100.69 71.29) (end 100.765001 71.365001) (width 0.25) (layer F.Cu) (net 6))
 (segment (start 101.995 74.235) (end 101.995 73.66) (width 0.25) (layer F.Cu) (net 6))
 (segment (start 105.334072 77.574072) (end 101.995 74.235) (width 0.25) (layer F.Cu) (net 6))
 (segment (start 111.80493 77.574072) (end 105.334072 77.574072) (width 0.25) (layer F.Cu) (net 6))
 (segment (start 111.045 56.275) (end 111.44 55.88) (width 0.25) (layer F.Cu) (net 7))
 (segment (start 97.99 66.79) (end 97.09 66.79) (width 0.25) (layer F.Cu) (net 7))
 (segment (start 98.99 66.79) (end 97.99 66.79) (width 0.25) (layer F.Cu) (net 7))
 (segment (start 101.69 69.49) (end 98.99 66.79) (width 0.25) (layer F.Cu) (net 7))
 (segment (start 101.69 70.39) (end 101.69 69.49) (width 0.25) (layer F.Cu) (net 7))
 (segment (start 105.41 55.88) (end 100.33 60.96) (width 0.25) (layer B.Cu) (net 7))
 (via (at 100.33 66.04) (size 0.8) (drill 0.4) (layers F.Cu B.Cu) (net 7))
 (segment (start 100.33 60.96) (end 100.33 66.04) (width 0.25) (layer B.Cu) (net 7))
 (segment (start 99.74 66.04) (end 98.99 66.79) (width 0.25) (layer F.Cu) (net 7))
 (segment (start 100.33 66.04) (end 99.74 66.04) (width 0.25) (layer F.Cu) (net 7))
 (segment (start 110.565 55.005) (end 111.44 55.88) (width 0.25) (layer F.Cu) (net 7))
 (segment (start 106.68 55.005) (end 110.565 55.005) (width 0.25) (layer F.Cu) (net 7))
 (segment (start 106.68 55.005) (end 106.285 55.005) (width 0.25) (layer F.Cu) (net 7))
 (via (at 105.41 55.88) (size 0.8) (drill 0.4) (layers F.Cu B.Cu) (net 7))
 (segment (start 106.285 55.005) (end 105.41 55.88) (width 0.25) (layer F.Cu) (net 7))
 (segment (start 104.19 73.215) (end 103.745 73.66) (width 0.25) (layer F.Cu) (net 8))
 (segment (start 104.19 70.39) (end 104.19 73.215) (width 0.25) (layer F.Cu) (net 8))
 (segment (start 99.69 72.145) (end 100.33 72.785) (width 0.25) (layer F.Cu) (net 9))
 (segment (start 99.69 70.39) (end 99.69 72.145) (width 0.25) (layer F.Cu) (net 9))
 (segment (start 98.69 71.29) (end 98.69 70.39) (width 0.25) (layer F.Cu) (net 10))
 (segment (start 98.69 71.79) (end 98.69 71.29) (width 0.25) (layer F.Cu) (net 10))
 (segment (start 99.06 72.16) (end 98.69 71.79) (width 0.25) (layer F.Cu) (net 10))
 (segment (start 99.06 72.785) (end 99.06 72.16) (width 0.25) (layer F.Cu) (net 10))
 (segment (start 97.09 64.79) (end 90.19 64.79) (width 0.25) (layer F.Cu) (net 11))
 (segment (start 90.19 64.79) (end 90.17 64.81) (width 0.25) (layer F.Cu) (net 11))
 (segment (start 90.17 69.85) (end 91.44 71.12) (width 0.25) (layer F.Cu) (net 11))
 (segment (start 90.17 64.81) (end 90.17 69.85) (width 0.25) (layer F.Cu) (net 11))
 (segment (start 96.19 65.79) (end 93.4 68.58) (width 0.25) (layer F.Cu) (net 12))
 (segment (start 97.09 65.79) (end 96.19 65.79) (width 0.25) (layer F.Cu) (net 12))
 (segment (start 93.4 68.58) (end 91.44 68.58) (width 0.25) (layer F.Cu) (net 12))
 (segment (start 92.19 65.29) (end 91.44 66.04) (width 0.25) (layer F.Cu) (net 13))
 (segment (start 97.09 65.29) (end 92.19 65.29) (width 0.25) (layer F.Cu) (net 13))
 (segment (start 92.23 64.29) (end 91.44 63.5) (width 0.25) (layer F.Cu) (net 14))
 (segment (start 97.09 64.29) (end 92.23 64.29) (width 0.25) (layer F.Cu) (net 14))
 (segment (start 94.27 63.79) (end 91.44 60.96) (width 0.25) (layer F.Cu) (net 15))
 (segment (start 97.09 63.79) (end 94.27 63.79) (width 0.25) (layer F.Cu) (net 15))
 (segment (start 97.09 63.29) (end 96.565 63.29) (width 0.25) (layer F.Cu) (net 16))
 (segment (start 97.09 63.29) (end 94.40641 63.29) (width 0.25) (layer F.Cu) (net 16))
 (segment (start 94.40641 63.29) (end 92.71 61.59359) (width 0.25) (layer F.Cu) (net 16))
 (segment (start 92.71 61.59359) (end 92.71 59.69) (width 0.25) (layer F.Cu) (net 16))
 (segment (start 92.71 59.69) (end 91.44 58.42) (width 0.25) (layer F.Cu) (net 16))
 (segment (start 91.44 55.88) (end 97.79 55.88) (width 0.25) (layer F.Cu) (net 17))
 (segment (start 99.69 59.50551) (end 100.33 58.86551) (width 0.25) (layer F.Cu) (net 17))
 (segment (start 99.69 61.69) (end 99.69 59.50551) (width 0.25) (layer F.Cu) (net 17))
 (segment (start 98.23551 55.88) (end 97.79 55.88) (width 0.25) (layer F.Cu) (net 17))
 (segment (start 100.33 57.97449) (end 98.23551 55.88) (width 0.25) (layer F.Cu) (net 17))
 (segment (start 100.33 58.86551) (end 100.33 57.97449) (width 0.25) (layer F.Cu) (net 17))
 (segment (start 105.41 76.2) (end 111.44 76.2) (width 0.25) (layer F.Cu) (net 18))
 (segment (start 103.19 70.39) (end 103.19 72.34001) (width 0.25) (layer F.Cu) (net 18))
 (segment (start 104.96449 76.2) (end 105.41 76.2) (width 0.25) (layer F.Cu) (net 18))
 (segment (start 102.87 74.10551) (end 104.96449 76.2) (width 0.25) (layer F.Cu) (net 18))
 (segment (start 102.87 72.66001) (end 102.87 74.10551) (width 0.25) (layer F.Cu) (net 18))
 (segment (start 103.19 72.34001) (end 102.87 72.66001) (width 0.25) (layer F.Cu) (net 18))
 (segment (start 105.79 68.79) (end 106.315 68.79) (width 0.25) (layer F.Cu) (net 19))
 (segment (start 106.47 68.79) (end 106.51999 68.74001) (width 0.25) (layer F.Cu) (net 19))
 (segment (start 105.79 68.79) (end 106.47 68.79) (width 0.25) (layer F.Cu) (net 19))
 (segment (start 106.51999 68.74001) (end 108.7436 68.74001) (width 0.25) (layer F.Cu) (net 19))
 (segment (start 110.590001 72.810001) (end 111.44 73.66) (width 0.25) (layer F.Cu) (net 19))
 (segment (start 110.03999 72.25999) (end 110.590001 72.810001) (width 0.25) (layer F.Cu) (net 19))
 (segment (start 110.03999 70.0364) (end 110.03999 72.25999) (width 0.25) (layer F.Cu) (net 19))
 (segment (start 108.7436 68.74001) (end 110.03999 70.0364) (width 0.25) (layer F.Cu) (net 19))
 (segment (start 110.49 70.17) (end 111.44 71.12) (width 0.25) (layer F.Cu) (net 20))
 (segment (start 110.49 69.85) (end 110.49 70.17) (width 0.25) (layer F.Cu) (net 20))
 (segment (start 105.79 68.29) (end 108.93 68.29) (width 0.25) (layer F.Cu) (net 20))
 (segment (start 108.93 68.29) (end 110.49 69.85) (width 0.25) (layer F.Cu) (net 20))
 (segment (start 110.65 67.79) (end 111.44 68.58) (width 0.25) (layer F.Cu) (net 21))
 (segment (start 105.79 67.79) (end 110.65 67.79) (width 0.25) (layer F.Cu) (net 21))
 (segment (start 110.69 66.79) (end 111.44 66.04) (width 0.25) (layer F.Cu) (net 22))
 (segment (start 105.79 66.79) (end 110.69 66.79) (width 0.25) (layer F.Cu) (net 22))
 (segment (start 106.69 66.29) (end 109.48 63.5) (width 0.25) (layer F.Cu) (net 23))
 (segment (start 105.79 66.29) (end 106.69 66.29) (width 0.25) (layer F.Cu) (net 23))
 (segment (start 109.48 63.5) (end 111.44 63.5) (width 0.25) (layer F.Cu) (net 23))
 (segment (start 112.289999 61.809999) (end 111.44 60.96) (width 0.25) (layer F.Cu) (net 24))
 (segment (start 112.615001 62.135001) (end 112.289999 61.809999) (width 0.25) (layer F.Cu) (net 24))
 (segment (start 112.615001 66.604001) (end 112.615001 62.135001) (width 0.25) (layer F.Cu) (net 24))
 (segment (start 111.929002 67.29) (end 112.615001 66.604001) (width 0.25) (layer F.Cu) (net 24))
 (segment (start 105.79 67.29) (end 111.929002 67.29) (width 0.25) (layer F.Cu) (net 24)))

